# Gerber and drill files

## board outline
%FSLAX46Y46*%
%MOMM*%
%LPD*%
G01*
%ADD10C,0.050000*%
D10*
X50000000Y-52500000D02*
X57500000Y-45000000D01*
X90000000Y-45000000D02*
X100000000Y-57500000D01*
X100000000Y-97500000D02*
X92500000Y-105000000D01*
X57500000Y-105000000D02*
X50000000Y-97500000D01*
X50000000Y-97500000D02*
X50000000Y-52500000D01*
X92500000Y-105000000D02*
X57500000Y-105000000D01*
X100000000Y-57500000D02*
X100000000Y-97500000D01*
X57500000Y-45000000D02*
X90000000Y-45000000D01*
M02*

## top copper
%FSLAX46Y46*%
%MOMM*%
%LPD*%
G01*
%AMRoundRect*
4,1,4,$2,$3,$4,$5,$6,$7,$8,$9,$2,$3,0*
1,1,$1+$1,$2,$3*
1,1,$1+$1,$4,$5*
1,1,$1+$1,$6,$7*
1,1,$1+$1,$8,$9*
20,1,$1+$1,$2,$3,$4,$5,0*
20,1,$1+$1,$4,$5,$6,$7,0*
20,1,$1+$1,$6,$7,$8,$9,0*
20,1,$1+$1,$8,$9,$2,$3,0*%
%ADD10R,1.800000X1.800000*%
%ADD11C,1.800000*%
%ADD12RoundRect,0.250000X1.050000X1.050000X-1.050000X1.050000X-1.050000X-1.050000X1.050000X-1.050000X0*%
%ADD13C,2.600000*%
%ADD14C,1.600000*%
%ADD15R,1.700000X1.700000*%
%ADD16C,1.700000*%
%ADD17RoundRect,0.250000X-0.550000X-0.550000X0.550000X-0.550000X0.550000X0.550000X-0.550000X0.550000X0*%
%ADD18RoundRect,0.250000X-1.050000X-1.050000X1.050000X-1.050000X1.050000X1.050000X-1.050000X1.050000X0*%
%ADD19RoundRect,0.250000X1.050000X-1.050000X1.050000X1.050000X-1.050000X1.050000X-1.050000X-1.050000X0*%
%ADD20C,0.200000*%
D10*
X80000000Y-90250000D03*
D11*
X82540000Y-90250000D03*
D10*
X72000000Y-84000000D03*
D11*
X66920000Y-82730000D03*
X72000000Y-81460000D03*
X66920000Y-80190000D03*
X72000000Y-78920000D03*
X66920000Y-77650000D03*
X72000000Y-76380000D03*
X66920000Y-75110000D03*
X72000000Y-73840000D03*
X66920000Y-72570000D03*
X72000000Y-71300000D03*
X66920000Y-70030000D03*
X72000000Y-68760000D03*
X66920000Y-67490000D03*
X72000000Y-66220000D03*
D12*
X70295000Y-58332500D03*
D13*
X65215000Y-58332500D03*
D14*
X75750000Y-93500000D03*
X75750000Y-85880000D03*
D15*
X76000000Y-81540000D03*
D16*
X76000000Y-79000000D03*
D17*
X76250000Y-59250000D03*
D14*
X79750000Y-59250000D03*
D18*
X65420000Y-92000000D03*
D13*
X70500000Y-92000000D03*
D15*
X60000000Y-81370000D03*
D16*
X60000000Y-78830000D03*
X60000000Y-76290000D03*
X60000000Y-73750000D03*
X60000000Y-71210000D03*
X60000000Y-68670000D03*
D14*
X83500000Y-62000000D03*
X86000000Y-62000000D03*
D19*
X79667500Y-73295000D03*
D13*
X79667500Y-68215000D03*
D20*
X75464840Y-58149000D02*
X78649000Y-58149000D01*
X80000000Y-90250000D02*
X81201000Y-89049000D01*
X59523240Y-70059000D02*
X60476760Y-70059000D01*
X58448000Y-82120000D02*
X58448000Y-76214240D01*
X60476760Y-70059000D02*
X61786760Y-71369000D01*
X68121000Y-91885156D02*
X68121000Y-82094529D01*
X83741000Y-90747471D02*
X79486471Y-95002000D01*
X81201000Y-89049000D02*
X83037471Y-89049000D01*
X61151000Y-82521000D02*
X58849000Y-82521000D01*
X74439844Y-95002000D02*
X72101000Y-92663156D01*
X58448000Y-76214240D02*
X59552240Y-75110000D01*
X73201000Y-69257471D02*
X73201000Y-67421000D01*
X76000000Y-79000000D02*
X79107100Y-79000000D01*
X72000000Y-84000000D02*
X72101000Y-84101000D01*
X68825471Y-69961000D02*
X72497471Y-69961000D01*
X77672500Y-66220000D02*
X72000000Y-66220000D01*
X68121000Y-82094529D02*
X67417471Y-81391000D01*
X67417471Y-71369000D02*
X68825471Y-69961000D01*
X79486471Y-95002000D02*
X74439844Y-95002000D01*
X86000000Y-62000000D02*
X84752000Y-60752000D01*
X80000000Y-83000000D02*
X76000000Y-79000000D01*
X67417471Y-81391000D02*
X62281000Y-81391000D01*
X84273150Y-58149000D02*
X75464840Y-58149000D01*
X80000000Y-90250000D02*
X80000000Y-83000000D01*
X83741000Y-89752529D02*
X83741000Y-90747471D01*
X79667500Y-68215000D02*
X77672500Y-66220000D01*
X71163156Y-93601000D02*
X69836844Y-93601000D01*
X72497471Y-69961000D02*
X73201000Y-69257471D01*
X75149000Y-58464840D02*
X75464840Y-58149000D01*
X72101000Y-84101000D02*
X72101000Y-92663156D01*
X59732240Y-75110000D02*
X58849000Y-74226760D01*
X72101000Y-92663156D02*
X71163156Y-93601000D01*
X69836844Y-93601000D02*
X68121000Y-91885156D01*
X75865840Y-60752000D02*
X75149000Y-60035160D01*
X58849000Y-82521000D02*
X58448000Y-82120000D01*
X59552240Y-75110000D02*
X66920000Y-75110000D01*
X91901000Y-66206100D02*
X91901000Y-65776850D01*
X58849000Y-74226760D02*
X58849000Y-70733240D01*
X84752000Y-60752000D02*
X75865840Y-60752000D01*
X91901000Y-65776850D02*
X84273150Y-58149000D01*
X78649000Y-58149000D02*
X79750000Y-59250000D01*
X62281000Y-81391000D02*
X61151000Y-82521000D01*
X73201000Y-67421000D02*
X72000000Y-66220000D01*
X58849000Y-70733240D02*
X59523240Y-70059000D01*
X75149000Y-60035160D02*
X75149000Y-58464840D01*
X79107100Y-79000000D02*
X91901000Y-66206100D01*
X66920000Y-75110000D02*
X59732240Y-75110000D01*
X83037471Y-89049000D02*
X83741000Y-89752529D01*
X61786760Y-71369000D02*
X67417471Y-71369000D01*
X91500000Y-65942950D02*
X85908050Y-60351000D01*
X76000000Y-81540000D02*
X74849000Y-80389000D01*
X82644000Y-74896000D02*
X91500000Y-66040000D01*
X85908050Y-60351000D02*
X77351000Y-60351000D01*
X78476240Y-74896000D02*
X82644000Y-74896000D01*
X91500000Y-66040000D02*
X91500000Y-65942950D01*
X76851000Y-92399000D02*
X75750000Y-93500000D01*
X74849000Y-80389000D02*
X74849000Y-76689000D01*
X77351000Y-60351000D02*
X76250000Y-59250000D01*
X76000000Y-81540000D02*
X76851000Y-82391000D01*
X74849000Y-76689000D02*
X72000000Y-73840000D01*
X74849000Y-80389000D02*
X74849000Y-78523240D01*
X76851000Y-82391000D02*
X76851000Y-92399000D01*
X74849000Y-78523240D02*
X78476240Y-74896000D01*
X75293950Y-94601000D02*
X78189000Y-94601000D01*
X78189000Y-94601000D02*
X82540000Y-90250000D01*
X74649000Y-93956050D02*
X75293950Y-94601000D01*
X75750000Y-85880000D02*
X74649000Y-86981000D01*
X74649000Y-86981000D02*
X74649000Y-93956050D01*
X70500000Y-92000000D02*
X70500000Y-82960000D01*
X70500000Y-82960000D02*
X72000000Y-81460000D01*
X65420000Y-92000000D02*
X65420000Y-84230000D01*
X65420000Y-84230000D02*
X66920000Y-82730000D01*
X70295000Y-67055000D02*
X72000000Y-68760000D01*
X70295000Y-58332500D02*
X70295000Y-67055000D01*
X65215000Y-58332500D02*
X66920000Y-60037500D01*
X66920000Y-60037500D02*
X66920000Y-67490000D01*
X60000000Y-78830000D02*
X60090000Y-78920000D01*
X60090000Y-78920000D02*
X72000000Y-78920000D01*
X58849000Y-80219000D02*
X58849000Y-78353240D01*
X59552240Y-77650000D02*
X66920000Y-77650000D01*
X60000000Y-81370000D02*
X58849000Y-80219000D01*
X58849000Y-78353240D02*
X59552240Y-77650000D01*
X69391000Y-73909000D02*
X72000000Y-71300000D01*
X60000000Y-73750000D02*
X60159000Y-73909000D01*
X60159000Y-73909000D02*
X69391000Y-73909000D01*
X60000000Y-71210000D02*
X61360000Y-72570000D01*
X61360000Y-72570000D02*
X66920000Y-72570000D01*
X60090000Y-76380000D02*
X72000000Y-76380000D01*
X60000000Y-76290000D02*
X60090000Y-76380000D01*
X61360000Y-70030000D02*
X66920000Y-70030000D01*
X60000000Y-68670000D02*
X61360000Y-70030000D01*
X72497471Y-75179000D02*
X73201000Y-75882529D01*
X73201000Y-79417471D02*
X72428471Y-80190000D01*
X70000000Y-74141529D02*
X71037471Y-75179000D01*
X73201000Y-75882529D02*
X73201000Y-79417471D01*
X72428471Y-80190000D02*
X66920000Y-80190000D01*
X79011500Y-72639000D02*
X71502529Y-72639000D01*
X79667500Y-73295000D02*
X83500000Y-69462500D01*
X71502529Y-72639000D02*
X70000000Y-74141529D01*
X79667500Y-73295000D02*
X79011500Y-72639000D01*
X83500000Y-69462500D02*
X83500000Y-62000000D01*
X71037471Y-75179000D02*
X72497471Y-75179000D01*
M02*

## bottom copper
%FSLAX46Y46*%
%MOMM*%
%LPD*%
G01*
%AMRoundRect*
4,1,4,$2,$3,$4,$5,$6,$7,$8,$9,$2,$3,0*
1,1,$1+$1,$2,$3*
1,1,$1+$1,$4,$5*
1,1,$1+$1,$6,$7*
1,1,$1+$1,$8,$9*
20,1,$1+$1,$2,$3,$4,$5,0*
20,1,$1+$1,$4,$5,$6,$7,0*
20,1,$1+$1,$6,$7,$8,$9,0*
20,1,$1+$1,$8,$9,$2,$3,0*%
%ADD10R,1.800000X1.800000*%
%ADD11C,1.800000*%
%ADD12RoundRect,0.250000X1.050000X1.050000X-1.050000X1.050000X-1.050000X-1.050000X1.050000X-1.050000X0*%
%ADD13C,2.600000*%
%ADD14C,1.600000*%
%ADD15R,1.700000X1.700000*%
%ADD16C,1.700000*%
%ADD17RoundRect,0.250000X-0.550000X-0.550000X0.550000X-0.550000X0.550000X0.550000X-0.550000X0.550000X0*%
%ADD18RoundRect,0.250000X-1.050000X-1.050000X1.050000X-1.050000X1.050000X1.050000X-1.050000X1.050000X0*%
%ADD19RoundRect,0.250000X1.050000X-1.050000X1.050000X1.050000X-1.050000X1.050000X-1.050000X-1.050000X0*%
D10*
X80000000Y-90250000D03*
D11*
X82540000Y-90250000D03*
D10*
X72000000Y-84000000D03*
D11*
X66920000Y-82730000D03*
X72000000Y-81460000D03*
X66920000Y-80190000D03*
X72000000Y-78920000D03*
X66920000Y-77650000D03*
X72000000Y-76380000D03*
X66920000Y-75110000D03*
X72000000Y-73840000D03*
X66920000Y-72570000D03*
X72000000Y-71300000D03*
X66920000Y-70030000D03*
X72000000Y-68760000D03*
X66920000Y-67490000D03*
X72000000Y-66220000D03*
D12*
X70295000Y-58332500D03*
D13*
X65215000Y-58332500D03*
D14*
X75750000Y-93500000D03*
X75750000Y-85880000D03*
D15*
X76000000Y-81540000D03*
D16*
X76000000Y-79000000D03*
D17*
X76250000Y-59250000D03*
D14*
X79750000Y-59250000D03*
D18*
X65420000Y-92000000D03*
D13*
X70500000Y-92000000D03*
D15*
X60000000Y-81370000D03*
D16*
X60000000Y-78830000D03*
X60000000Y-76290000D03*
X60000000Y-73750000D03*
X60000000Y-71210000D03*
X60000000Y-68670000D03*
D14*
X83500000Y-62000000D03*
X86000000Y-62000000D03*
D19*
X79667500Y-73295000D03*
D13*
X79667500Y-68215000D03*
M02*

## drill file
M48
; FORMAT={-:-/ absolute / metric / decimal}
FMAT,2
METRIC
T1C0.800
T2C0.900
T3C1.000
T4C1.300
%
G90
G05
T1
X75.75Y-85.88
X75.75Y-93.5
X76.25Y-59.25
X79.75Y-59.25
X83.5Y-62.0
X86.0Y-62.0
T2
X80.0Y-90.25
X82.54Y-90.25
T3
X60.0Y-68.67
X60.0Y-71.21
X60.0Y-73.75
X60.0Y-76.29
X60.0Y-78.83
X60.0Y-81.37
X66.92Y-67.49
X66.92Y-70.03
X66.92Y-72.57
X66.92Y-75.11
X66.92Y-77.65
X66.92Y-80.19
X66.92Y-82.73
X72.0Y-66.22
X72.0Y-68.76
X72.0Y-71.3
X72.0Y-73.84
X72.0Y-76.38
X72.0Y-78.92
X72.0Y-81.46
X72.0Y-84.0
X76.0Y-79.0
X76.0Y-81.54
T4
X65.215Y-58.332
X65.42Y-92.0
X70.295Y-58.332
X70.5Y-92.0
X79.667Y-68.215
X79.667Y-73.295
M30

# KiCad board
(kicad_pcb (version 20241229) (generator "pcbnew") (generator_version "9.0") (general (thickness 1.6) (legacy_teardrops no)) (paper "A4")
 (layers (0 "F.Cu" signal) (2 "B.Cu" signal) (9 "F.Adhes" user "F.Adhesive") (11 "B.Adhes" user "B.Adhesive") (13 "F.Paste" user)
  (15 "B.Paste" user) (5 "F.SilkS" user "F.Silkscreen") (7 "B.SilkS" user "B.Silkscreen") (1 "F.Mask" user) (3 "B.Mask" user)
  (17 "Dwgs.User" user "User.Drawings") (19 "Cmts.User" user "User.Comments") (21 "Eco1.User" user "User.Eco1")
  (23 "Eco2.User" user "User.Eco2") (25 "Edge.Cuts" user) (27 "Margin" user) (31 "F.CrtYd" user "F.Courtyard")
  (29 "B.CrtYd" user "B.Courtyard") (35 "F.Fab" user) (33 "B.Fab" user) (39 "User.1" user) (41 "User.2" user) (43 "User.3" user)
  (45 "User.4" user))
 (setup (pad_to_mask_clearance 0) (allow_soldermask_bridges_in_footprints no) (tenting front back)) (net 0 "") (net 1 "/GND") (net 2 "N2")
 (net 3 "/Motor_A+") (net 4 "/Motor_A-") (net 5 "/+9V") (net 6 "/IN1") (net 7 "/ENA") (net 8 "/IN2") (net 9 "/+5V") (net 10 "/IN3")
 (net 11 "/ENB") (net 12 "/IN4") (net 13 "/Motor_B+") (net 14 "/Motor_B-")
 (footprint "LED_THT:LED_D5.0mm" (layer "F.Cu") (at 80 90.25)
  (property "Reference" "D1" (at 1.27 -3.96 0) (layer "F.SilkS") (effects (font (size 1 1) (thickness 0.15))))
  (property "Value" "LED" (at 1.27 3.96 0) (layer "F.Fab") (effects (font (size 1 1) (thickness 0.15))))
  (pad "1" thru_hole rect (at 0 0) (size 1.8 1.8) (drill 0.9) (layers "*.Cu" "*.Mask") (remove_unused_layers no) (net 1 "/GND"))
  (pad "2" thru_hole circle (at 2.54 0) (size 1.8 1.8) (drill 0.9) (layers "*.Cu" "*.Mask") (remove_unused_layers no) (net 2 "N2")))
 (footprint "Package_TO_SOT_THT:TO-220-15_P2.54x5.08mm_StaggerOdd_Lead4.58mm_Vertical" (layer "F.Cu") (at 72 84 90)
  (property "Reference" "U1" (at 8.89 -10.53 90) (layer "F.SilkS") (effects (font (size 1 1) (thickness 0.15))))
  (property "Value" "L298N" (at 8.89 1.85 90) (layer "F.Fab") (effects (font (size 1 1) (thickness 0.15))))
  (pad "1" thru_hole rect (at 0 0 90) (size 1.8 1.8) (drill 1) (layers "*.Cu" "*.Mask") (remove_unused_layers no) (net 1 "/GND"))
  (pad "2" thru_hole circle (at 1.27 -5.08 90) (size 1.8 1.8) (drill 1) (layers "*.Cu" "*.Mask") (remove_unused_layers no)
   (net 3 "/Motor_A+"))
  (pad "3" thru_hole circle (at 2.54 0 90) (size 1.8 1.8) (drill 1) (layers "*.Cu" "*.Mask") (remove_unused_layers no) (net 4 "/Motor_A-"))
  (pad "4" thru_hole circle (at 3.81 -5.08 90) (size 1.8 1.8) (drill 1) (layers "*.Cu" "*.Mask") (remove_unused_layers no) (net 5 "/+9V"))
  (pad "5" thru_hole circle (at 5.08 0 90) (size 1.8 1.8) (drill 1) (layers "*.Cu" "*.Mask") (remove_unused_layers no) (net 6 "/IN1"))
  (pad "6" thru_hole circle (at 6.35 -5.08 90) (size 1.8 1.8) (drill 1) (layers "*.Cu" "*.Mask") (remove_unused_layers no) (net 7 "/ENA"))
  (pad "7" thru_hole circle (at 7.62 0 90) (size 1.8 1.8) (drill 1) (layers "*.Cu" "*.Mask") (remove_unused_layers no) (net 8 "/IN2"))
  (pad "8" thru_hole circle (at 8.89 -5.08 90) (size 1.8 1.8) (drill 1) (layers "*.Cu" "*.Mask") (remove_unused_layers no) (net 1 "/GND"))
  (pad "9" thru_hole circle (at 10.16 0 90) (size 1.8 1.8) (drill 1) (layers "*.Cu" "*.Mask") (remove_unused_layers no) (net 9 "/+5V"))
  (pad "10" thru_hole circle (at 11.43 -5.08 90) (size 1.8 1.8) (drill 1) (layers "*.Cu" "*.Mask") (remove_unused_layers no) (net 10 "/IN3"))
  (pad "11" thru_hole circle (at 12.7 0 90) (size 1.8 1.8) (drill 1) (layers "*.Cu" "*.Mask") (remove_unused_layers no) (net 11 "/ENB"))
  (pad "12" thru_hole circle (at 13.97 -5.08 90) (size 1.8 1.8) (drill 1) (layers "*.Cu" "*.Mask") (remove_unused_layers no) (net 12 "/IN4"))
  (pad "13" thru_hole circle (at 15.24 0 90) (size 1.8 1.8) (drill 1) (layers "*.Cu" "*.Mask") (remove_unused_layers no)
   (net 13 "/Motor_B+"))
  (pad "14" thru_hole circle (at 16.51 -5.08 90) (size 1.8 1.8) (drill 1) (layers "*.Cu" "*.Mask") (remove_unused_layers no)
   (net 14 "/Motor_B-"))
  (pad "15" thru_hole circle (at 17.78 0 90) (size 1.8 1.8) (drill 1) (layers "*.Cu" "*.Mask") (remove_unused_layers no) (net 1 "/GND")))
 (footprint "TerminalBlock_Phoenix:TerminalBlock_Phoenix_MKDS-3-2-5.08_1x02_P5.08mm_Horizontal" (layer "F.Cu") (at 70.295 58.3325 180)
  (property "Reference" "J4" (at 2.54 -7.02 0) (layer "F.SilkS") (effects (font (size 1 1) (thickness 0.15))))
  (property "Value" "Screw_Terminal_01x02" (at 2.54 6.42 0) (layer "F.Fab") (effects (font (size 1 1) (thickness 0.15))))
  (pad "1" thru_hole roundrect (at 0 0 180) (size 2.6 2.6) (drill 1.3) (layers "*.Cu" "*.Mask") (remove_unused_layers no)
   (roundrect_rratio 0.096154) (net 13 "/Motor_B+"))
  (pad "2" thru_hole circle (at 5.08 0 180) (size 2.6 2.6) (drill 1.3) (layers "*.Cu" "*.Mask") (remove_unused_layers no)
   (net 14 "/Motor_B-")))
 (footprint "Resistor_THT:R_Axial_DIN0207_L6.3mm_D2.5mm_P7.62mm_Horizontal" (layer "F.Cu") (at 75.75 93.5 90)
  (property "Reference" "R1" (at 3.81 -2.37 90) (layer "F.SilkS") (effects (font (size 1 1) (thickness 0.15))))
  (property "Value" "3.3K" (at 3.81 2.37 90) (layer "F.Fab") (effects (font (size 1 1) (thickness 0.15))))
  (pad "1" thru_hole circle (at 0 0 90) (size 1.6 1.6) (drill 0.8) (layers "*.Cu" "*.Mask") (remove_unused_layers no) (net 9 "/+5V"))
  (pad "2" thru_hole circle (at 7.62 0 90) (size 1.6 1.6) (drill 0.8) (layers "*.Cu" "*.Mask") (remove_unused_layers no) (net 2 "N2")))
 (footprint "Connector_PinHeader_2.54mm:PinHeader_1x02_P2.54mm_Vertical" (layer "F.Cu") (at 76 81.54 180)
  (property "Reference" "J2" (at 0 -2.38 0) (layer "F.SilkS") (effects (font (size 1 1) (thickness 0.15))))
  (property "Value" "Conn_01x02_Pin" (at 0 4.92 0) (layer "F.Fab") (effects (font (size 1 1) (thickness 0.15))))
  (pad "1" thru_hole rect (at 0 0 180) (size 1.7 1.7) (drill 1) (layers "*.Cu" "*.Mask") (remove_unused_layers no) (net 9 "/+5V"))
  (pad "2" thru_hole circle (at 0 2.54 180) (size 1.7 1.7) (drill 1) (layers "*.Cu" "*.Mask") (remove_unused_layers no) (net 1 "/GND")))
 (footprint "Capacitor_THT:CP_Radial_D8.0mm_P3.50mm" (layer "F.Cu") (at 76.25 59.25)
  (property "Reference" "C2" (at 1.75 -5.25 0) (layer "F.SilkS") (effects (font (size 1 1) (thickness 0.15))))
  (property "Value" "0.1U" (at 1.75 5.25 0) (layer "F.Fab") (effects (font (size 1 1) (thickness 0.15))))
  (pad "1" thru_hole roundrect (at 0 0) (size 1.6 1.6) (drill 0.8) (layers "*.Cu" "*.Mask") (remove_unused_layers no)
   (roundrect_rratio 0.15625) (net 9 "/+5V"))
  (pad "2" thru_hole circle (at 3.5 0) (size 1.6 1.6) (drill 0.8) (layers "*.Cu" "*.Mask") (remove_unused_layers no) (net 1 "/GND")))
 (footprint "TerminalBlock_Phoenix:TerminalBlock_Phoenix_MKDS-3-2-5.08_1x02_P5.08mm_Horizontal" (layer "F.Cu") (at 65.42 92)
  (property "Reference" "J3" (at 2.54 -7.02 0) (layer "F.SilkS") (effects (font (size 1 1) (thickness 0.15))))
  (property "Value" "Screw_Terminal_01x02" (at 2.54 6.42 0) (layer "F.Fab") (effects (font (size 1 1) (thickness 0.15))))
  (pad "1" thru_hole roundrect (at 0 0) (size 2.6 2.6) (drill 1.3) (layers "*.Cu" "*.Mask") (remove_unused_layers no)
   (roundrect_rratio 0.096154) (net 3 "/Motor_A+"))
  (pad "2" thru_hole circle (at 5.08 0) (size 2.6 2.6) (drill 1.3) (layers "*.Cu" "*.Mask") (remove_unused_layers no) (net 4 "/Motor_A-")))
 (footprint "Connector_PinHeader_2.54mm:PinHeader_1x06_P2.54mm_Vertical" (layer "F.Cu") (at 60 81.37 180)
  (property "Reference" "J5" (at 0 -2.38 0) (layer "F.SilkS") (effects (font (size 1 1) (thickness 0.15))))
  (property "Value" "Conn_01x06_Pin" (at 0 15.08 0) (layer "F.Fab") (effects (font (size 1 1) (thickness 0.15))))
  (pad "1" thru_hole rect (at 0 0 180) (size 1.7 1.7) (drill 1) (layers "*.Cu" "*.Mask") (remove_unused_layers no) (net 7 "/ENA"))
  (pad "2" thru_hole circle (at 0 2.54 180) (size 1.7 1.7) (drill 1) (layers "*.Cu" "*.Mask") (remove_unused_layers no) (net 6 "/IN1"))
  (pad "3" thru_hole circle (at 0 5.08 180) (size 1.7 1.7) (drill 1) (layers "*.Cu" "*.Mask") (remove_unused_layers no) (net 8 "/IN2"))
  (pad "4" thru_hole circle (at 0 7.62 180) (size 1.7 1.7) (drill 1) (layers "*.Cu" "*.Mask") (remove_unused_layers no) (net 11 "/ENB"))
  (pad "5" thru_hole circle (at 0 10.16 180) (size 1.7 1.7) (drill 1) (layers "*.Cu" "*.Mask") (remove_unused_layers no) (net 10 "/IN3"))
  (pad "6" thru_hole circle (at 0 12.7 180) (size 1.7 1.7) (drill 1) (layers "*.Cu" "*.Mask") (remove_unused_layers no) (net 12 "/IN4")))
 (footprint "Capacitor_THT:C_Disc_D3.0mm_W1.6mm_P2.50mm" (layer "F.Cu") (at 83.5 62)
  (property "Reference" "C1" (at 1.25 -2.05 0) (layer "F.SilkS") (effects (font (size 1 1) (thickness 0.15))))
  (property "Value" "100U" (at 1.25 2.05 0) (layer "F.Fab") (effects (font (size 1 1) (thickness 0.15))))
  (pad "1" thru_hole circle (at 0 0) (size 1.6 1.6) (drill 0.8) (layers "*.Cu" "*.Mask") (remove_unused_layers no) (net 5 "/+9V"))
  (pad "2" thru_hole circle (at 2.5 0) (size 1.6 1.6) (drill 0.8) (layers "*.Cu" "*.Mask") (remove_unused_layers no) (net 1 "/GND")))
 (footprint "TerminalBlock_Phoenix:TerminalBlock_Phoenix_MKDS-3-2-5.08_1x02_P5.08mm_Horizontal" (layer "F.Cu") (at 79.6675 73.295 90)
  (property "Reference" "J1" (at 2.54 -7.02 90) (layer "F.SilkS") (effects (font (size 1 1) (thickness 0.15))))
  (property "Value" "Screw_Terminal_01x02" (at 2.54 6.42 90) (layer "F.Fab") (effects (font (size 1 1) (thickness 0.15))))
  (pad "1" thru_hole roundrect (at 0 0 90) (size 2.6 2.6) (drill 1.3) (layers "*.Cu" "*.Mask") (remove_unused_layers no)
   (roundrect_rratio 0.096154) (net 5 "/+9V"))
  (pad "2" thru_hole circle (at 5.08 0 90) (size 2.6 2.6) (drill 1.3) (layers "*.Cu" "*.Mask") (remove_unused_layers no) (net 1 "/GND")))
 (gr_line (start 50 52.5) (end 57.5 45) (stroke (width 0.05) (type default)) (layer "Edge.Cuts"))
 (gr_line (start 90 45) (end 100 57.5) (stroke (width 0.05) (type default)) (layer "Edge.Cuts"))
 (gr_line (start 100 97.5) (end 92.5 105) (stroke (width 0.05) (type default)) (layer "Edge.Cuts"))
 (gr_line (start 57.5 105) (end 50 97.5) (stroke (width 0.05) (type default)) (layer "Edge.Cuts"))
 (gr_line (start 50 97.5) (end 50 52.5) (stroke (width 0.05) (type default)) (layer "Edge.Cuts"))
 (gr_line (start 92.5 105) (end 57.5 105) (stroke (width 0.05) (type default)) (layer "Edge.Cuts"))
 (gr_line (start 100 57.5) (end 100 97.5) (stroke (width 0.05) (type default)) (layer "Edge.Cuts"))
 (gr_line (start 57.5 45) (end 90 45) (stroke (width 0.05) (type default)) (layer "Edge.Cuts"))
 (segment (start 75.46484 58.149) (end 78.649 58.149) (width 0.2) (layer "F.Cu") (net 1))
 (segment (start 80 90.25) (end 81.201 89.049) (width 0.2) (layer "F.Cu") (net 1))
 (segment (start 59.52324 70.059) (end 60.47676 70.059) (width 0.2) (layer "F.Cu") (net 1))
 (segment (start 58.448 82.12) (end 58.448 76.21424) (width 0.2) (layer "F.Cu") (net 1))
 (segment (start 60.47676 70.059) (end 61.78676 71.369) (width 0.2) (layer "F.Cu") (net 1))
 (segment (start 68.121 91.885156) (end 68.121 82.094529) (width 0.2) (layer "F.Cu") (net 1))
 (segment (start 83.741 90.747471) (end 79.486471 95.002) (width 0.2) (layer "F.Cu") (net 1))
 (segment (start 81.201 89.049) (end 83.037471 89.049) (width 0.2) (layer "F.Cu") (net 1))
 (segment (start 61.151 82.521) (end 58.849 82.521) (width 0.2) (layer "F.Cu") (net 1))
 (segment (start 74.439844 95.002) (end 72.101 92.663156) (width 0.2) (layer "F.Cu") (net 1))
 (segment (start 58.448 76.21424) (end 59.55224 75.11) (width 0.2) (layer "F.Cu") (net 1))
 (segment (start 73.201 69.257471) (end 73.201 67.421) (width 0.2) (layer "F.Cu") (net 1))
 (segment (start 76 79) (end 79.1071 79) (width 0.2) (layer "F.Cu") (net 1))
 (segment (start 72 84) (end 72.101 84.101) (width 0.2) (layer "F.Cu") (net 1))
 (segment (start 68.825471 69.961) (end 72.497471 69.961) (width 0.2) (layer "F.Cu") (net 1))
 (segment (start 77.6725 66.22) (end 72 66.22) (width 0.2) (layer "F.Cu") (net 1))
 (segment (start 68.121 82.094529) (end 67.417471 81.391) (width 0.2) (layer "F.Cu") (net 1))
 (segment (start 67.417471 71.369) (end 68.825471 69.961) (width 0.2) (layer "F.Cu") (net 1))
 (segment (start 79.486471 95.002) (end 74.439844 95.002) (width 0.2) (layer "F.Cu") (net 1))
 (segment (start 86 62) (end 84.752 60.752) (width 0.2) (layer "F.Cu") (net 1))
 (segment (start 80 83) (end 76 79) (width 0.2) (layer "F.Cu") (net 1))
 (segment (start 67.417471 81.391) (end 62.281 81.391) (width 0.2) (layer "F.Cu") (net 1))
 (segment (start 84.27315 58.149) (end 75.46484 58.149) (width 0.2) (layer "F.Cu") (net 1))
 (segment (start 80 90.25) (end 80 83) (width 0.2) (layer "F.Cu") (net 1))
 (segment (start 83.741 89.752529) (end 83.741 90.747471) (width 0.2) (layer "F.Cu") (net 1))
 (segment (start 79.6675 68.215) (end 77.6725 66.22) (width 0.2) (layer "F.Cu") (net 1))
 (segment (start 71.163156 93.601) (end 69.836844 93.601) (width 0.2) (layer "F.Cu") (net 1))
 (segment (start 72.497471 69.961) (end 73.201 69.257471) (width 0.2) (layer "F.Cu") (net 1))
 (segment (start 75.149 58.46484) (end 75.46484 58.149) (width 0.2) (layer "F.Cu") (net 1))
 (segment (start 72.101 84.101) (end 72.101 92.663156) (width 0.2) (layer "F.Cu") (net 1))
 (segment (start 59.73224 75.11) (end 58.849 74.22676) (width 0.2) (layer "F.Cu") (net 1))
 (segment (start 72.101 92.663156) (end 71.163156 93.601) (width 0.2) (layer "F.Cu") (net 1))
 (segment (start 69.836844 93.601) (end 68.121 91.885156) (width 0.2) (layer "F.Cu") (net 1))
 (segment (start 75.86584 60.752) (end 75.149 60.03516) (width 0.2) (layer "F.Cu") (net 1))
 (segment (start 58.849 82.521) (end 58.448 82.12) (width 0.2) (layer "F.Cu") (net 1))
 (segment (start 59.55224 75.11) (end 66.92 75.11) (width 0.2) (layer "F.Cu") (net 1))
 (segment (start 91.901 66.2061) (end 91.901 65.77685) (width 0.2) (layer "F.Cu") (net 1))
 (segment (start 58.849 74.22676) (end 58.849 70.73324) (width 0.2) (layer "F.Cu") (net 1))
 (segment (start 84.752 60.752) (end 75.86584 60.752) (width 0.2) (layer "F.Cu") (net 1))
 (segment (start 91.901 65.77685) (end 84.27315 58.149) (width 0.2) (layer "F.Cu") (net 1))
 (segment (start 78.649 58.149) (end 79.75 59.25) (width 0.2) (layer "F.Cu") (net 1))
 (segment (start 62.281 81.391) (end 61.151 82.521) (width 0.2) (layer "F.Cu") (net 1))
 (segment (start 73.201 67.421) (end 72 66.22) (width 0.2) (layer "F.Cu") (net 1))
 (segment (start 58.849 70.73324) (end 59.52324 70.059) (width 0.2) (layer "F.Cu") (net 1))
 (segment (start 75.149 60.03516) (end 75.149 58.46484) (width 0.2) (layer "F.Cu") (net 1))
 (segment (start 79.1071 79) (end 91.901 66.2061) (width 0.2) (layer "F.Cu") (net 1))
 (segment (start 66.92 75.11) (end 59.73224 75.11) (width 0.2) (layer "F.Cu") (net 1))
 (segment (start 83.037471 89.049) (end 83.741 89.752529) (width 0.2) (layer "F.Cu") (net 1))
 (segment (start 61.78676 71.369) (end 67.417471 71.369) (width 0.2) (layer "F.Cu") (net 1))
 (segment (start 91.5 65.94295) (end 85.90805 60.351) (width 0.2) (layer "F.Cu") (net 9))
 (segment (start 76 81.54) (end 74.849 80.389) (width 0.2) (layer "F.Cu") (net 9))
 (segment (start 82.644 74.896) (end 91.5 66.04) (width 0.2) (layer "F.Cu") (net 9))
 (segment (start 85.90805 60.351) (end 77.351 60.351) (width 0.2) (layer "F.Cu") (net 9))
 (segment (start 78.47624 74.896) (end 82.644 74.896) (width 0.2) (layer "F.Cu") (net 9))
 (segment (start 91.5 66.04) (end 91.5 65.94295) (width 0.2) (layer "F.Cu") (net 9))
 (segment (start 76.851 92.399) (end 75.75 93.5) (width 0.2) (layer "F.Cu") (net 9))
 (segment (start 74.849 80.389) (end 74.849 76.689) (width 0.2) (layer "F.Cu") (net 9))
 (segment (start 77.351 60.351) (end 76.25 59.25) (width 0.2) (layer "F.Cu") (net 9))
 (segment (start 76 81.54) (end 76.851 82.391) (width 0.2) (layer "F.Cu") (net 9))
 (segment (start 74.849 76.689) (end 72 73.84) (width 0.2) (layer "F.Cu") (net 9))
 (segment (start 74.849 80.389) (end 74.849 78.52324) (width 0.2) (layer "F.Cu") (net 9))
 (segment (start 76.851 82.391) (end 76.851 92.399) (width 0.2) (layer "F.Cu") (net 9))
 (segment (start 74.849 78.52324) (end 78.47624 74.896) (width 0.2) (layer "F.Cu") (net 9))
 (segment (start 75.29395 94.601) (end 78.189 94.601) (width 0.2) (layer "F.Cu") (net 2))
 (segment (start 78.189 94.601) (end 82.54 90.25) (width 0.2) (layer "F.Cu") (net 2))
 (segment (start 74.649 93.95605) (end 75.29395 94.601) (width 0.2) (layer "F.Cu") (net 2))
 (segment (start 75.75 85.88) (end 74.649 86.981) (width 0.2) (layer "F.Cu") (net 2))
 (segment (start 74.649 86.981) (end 74.649 93.95605) (width 0.2) (layer "F.Cu") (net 2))
 (segment (start 70.5 92) (end 70.5 82.96) (width 0.2) (layer "F.Cu") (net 4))
 (segment (start 70.5 82.96) (end 72 81.46) (width 0.2) (layer "F.Cu") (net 4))
 (segment (start 65.42 92) (end 65.42 84.23) (width 0.2) (layer "F.Cu") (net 3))
 (segment (start 65.42 84.23) (end 66.92 82.73) (width 0.2) (layer "F.Cu") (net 3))
 (segment (start 70.295 67.055) (end 72 68.76) (width 0.2) (layer "F.Cu") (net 13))
 (segment (start 70.295 58.3325) (end 70.295 67.055) (width 0.2) (layer "F.Cu") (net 13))
 (segment (start 65.215 58.3325) (end 66.92 60.0375) (width 0.2) (layer "F.Cu") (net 14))
 (segment (start 66.92 60.0375) (end 66.92 67.49) (width 0.2) (layer "F.Cu") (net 14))
 (segment (start 60 78.83) (end 60.09 78.92) (width 0.2) (layer "F.Cu") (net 6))
 (segment (start 60.09 78.92) (end 72 78.92) (width 0.2) (layer "F.Cu") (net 6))
 (segment (start 58.849 80.219) (end 58.849 78.35324) (width 0.2) (layer "F.Cu") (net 7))
 (segment (start 59.55224 77.65) (end 66.92 77.65) (width 0.2) (layer "F.Cu") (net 7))
 (segment (start 60 81.37) (end 58.849 80.219) (width 0.2) (layer "F.Cu") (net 7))
 (segment (start 58.849 78.35324) (end 59.55224 77.65) (width 0.2) (layer "F.Cu") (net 7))
 (segment (start 69.391 73.909) (end 72 71.3) (width 0.2) (layer "F.Cu") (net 11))
 (segment (start 60 73.75) (end 60.159 73.909) (width 0.2) (layer "F.Cu") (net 11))
 (segment (start 60.159 73.909) (end 69.391 73.909) (width 0.2) (layer "F.Cu") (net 11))
 (segment (start 60 71.21) (end 61.36 72.57) (width 0.2) (layer "F.Cu") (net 10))
 (segment (start 61.36 72.57) (end 66.92 72.57) (width 0.2) (layer "F.Cu") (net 10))
 (segment (start 60.09 76.38) (end 72 76.38) (width 0.2) (layer "F.Cu") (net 8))
 (segment (start 60 76.29) (end 60.09 76.38) (width 0.2) (layer "F.Cu") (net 8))
 (segment (start 61.36 70.03) (end 66.92 70.03) (width 0.2) (layer "F.Cu") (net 12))
 (segment (start 60 68.67) (end 61.36 70.03) (width 0.2) (layer "F.Cu") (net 12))
 (segment (start 72.497471 75.179) (end 73.201 75.882529) (width 0.2) (layer "F.Cu") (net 5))
 (segment (start 73.201 79.417471) (end 72.428471 80.19) (width 0.2) (layer "F.Cu") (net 5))
 (segment (start 70 74.141529) (end 71.037471 75.179) (width 0.2) (layer "F.Cu") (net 5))
 (segment (start 73.201 75.882529) (end 73.201 79.417471) (width 0.2) (layer "F.Cu") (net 5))
 (segment (start 72.428471 80.19) (end 66.92 80.19) (width 0.2) (layer "F.Cu") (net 5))
 (segment (start 79.0115 72.639) (end 71.502529 72.639) (width 0.2) (layer "F.Cu") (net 5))
 (segment (start 79.6675 73.295) (end 83.5 69.4625) (width 0.2) (layer "F.Cu") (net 5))
 (segment (start 71.502529 72.639) (end 70 74.141529) (width 0.2) (layer "F.Cu") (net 5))
 (segment (start 79.6675 73.295) (end 79.0115 72.639) (width 0.2) (layer "F.Cu") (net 5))
 (segment (start 83.5 69.4625) (end 83.5 62) (width 0.2) (layer "F.Cu") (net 5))
 (segment (start 71.037471 75.179) (end 72.497471 75.179) (width 0.2) (layer "F.Cu") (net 5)))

